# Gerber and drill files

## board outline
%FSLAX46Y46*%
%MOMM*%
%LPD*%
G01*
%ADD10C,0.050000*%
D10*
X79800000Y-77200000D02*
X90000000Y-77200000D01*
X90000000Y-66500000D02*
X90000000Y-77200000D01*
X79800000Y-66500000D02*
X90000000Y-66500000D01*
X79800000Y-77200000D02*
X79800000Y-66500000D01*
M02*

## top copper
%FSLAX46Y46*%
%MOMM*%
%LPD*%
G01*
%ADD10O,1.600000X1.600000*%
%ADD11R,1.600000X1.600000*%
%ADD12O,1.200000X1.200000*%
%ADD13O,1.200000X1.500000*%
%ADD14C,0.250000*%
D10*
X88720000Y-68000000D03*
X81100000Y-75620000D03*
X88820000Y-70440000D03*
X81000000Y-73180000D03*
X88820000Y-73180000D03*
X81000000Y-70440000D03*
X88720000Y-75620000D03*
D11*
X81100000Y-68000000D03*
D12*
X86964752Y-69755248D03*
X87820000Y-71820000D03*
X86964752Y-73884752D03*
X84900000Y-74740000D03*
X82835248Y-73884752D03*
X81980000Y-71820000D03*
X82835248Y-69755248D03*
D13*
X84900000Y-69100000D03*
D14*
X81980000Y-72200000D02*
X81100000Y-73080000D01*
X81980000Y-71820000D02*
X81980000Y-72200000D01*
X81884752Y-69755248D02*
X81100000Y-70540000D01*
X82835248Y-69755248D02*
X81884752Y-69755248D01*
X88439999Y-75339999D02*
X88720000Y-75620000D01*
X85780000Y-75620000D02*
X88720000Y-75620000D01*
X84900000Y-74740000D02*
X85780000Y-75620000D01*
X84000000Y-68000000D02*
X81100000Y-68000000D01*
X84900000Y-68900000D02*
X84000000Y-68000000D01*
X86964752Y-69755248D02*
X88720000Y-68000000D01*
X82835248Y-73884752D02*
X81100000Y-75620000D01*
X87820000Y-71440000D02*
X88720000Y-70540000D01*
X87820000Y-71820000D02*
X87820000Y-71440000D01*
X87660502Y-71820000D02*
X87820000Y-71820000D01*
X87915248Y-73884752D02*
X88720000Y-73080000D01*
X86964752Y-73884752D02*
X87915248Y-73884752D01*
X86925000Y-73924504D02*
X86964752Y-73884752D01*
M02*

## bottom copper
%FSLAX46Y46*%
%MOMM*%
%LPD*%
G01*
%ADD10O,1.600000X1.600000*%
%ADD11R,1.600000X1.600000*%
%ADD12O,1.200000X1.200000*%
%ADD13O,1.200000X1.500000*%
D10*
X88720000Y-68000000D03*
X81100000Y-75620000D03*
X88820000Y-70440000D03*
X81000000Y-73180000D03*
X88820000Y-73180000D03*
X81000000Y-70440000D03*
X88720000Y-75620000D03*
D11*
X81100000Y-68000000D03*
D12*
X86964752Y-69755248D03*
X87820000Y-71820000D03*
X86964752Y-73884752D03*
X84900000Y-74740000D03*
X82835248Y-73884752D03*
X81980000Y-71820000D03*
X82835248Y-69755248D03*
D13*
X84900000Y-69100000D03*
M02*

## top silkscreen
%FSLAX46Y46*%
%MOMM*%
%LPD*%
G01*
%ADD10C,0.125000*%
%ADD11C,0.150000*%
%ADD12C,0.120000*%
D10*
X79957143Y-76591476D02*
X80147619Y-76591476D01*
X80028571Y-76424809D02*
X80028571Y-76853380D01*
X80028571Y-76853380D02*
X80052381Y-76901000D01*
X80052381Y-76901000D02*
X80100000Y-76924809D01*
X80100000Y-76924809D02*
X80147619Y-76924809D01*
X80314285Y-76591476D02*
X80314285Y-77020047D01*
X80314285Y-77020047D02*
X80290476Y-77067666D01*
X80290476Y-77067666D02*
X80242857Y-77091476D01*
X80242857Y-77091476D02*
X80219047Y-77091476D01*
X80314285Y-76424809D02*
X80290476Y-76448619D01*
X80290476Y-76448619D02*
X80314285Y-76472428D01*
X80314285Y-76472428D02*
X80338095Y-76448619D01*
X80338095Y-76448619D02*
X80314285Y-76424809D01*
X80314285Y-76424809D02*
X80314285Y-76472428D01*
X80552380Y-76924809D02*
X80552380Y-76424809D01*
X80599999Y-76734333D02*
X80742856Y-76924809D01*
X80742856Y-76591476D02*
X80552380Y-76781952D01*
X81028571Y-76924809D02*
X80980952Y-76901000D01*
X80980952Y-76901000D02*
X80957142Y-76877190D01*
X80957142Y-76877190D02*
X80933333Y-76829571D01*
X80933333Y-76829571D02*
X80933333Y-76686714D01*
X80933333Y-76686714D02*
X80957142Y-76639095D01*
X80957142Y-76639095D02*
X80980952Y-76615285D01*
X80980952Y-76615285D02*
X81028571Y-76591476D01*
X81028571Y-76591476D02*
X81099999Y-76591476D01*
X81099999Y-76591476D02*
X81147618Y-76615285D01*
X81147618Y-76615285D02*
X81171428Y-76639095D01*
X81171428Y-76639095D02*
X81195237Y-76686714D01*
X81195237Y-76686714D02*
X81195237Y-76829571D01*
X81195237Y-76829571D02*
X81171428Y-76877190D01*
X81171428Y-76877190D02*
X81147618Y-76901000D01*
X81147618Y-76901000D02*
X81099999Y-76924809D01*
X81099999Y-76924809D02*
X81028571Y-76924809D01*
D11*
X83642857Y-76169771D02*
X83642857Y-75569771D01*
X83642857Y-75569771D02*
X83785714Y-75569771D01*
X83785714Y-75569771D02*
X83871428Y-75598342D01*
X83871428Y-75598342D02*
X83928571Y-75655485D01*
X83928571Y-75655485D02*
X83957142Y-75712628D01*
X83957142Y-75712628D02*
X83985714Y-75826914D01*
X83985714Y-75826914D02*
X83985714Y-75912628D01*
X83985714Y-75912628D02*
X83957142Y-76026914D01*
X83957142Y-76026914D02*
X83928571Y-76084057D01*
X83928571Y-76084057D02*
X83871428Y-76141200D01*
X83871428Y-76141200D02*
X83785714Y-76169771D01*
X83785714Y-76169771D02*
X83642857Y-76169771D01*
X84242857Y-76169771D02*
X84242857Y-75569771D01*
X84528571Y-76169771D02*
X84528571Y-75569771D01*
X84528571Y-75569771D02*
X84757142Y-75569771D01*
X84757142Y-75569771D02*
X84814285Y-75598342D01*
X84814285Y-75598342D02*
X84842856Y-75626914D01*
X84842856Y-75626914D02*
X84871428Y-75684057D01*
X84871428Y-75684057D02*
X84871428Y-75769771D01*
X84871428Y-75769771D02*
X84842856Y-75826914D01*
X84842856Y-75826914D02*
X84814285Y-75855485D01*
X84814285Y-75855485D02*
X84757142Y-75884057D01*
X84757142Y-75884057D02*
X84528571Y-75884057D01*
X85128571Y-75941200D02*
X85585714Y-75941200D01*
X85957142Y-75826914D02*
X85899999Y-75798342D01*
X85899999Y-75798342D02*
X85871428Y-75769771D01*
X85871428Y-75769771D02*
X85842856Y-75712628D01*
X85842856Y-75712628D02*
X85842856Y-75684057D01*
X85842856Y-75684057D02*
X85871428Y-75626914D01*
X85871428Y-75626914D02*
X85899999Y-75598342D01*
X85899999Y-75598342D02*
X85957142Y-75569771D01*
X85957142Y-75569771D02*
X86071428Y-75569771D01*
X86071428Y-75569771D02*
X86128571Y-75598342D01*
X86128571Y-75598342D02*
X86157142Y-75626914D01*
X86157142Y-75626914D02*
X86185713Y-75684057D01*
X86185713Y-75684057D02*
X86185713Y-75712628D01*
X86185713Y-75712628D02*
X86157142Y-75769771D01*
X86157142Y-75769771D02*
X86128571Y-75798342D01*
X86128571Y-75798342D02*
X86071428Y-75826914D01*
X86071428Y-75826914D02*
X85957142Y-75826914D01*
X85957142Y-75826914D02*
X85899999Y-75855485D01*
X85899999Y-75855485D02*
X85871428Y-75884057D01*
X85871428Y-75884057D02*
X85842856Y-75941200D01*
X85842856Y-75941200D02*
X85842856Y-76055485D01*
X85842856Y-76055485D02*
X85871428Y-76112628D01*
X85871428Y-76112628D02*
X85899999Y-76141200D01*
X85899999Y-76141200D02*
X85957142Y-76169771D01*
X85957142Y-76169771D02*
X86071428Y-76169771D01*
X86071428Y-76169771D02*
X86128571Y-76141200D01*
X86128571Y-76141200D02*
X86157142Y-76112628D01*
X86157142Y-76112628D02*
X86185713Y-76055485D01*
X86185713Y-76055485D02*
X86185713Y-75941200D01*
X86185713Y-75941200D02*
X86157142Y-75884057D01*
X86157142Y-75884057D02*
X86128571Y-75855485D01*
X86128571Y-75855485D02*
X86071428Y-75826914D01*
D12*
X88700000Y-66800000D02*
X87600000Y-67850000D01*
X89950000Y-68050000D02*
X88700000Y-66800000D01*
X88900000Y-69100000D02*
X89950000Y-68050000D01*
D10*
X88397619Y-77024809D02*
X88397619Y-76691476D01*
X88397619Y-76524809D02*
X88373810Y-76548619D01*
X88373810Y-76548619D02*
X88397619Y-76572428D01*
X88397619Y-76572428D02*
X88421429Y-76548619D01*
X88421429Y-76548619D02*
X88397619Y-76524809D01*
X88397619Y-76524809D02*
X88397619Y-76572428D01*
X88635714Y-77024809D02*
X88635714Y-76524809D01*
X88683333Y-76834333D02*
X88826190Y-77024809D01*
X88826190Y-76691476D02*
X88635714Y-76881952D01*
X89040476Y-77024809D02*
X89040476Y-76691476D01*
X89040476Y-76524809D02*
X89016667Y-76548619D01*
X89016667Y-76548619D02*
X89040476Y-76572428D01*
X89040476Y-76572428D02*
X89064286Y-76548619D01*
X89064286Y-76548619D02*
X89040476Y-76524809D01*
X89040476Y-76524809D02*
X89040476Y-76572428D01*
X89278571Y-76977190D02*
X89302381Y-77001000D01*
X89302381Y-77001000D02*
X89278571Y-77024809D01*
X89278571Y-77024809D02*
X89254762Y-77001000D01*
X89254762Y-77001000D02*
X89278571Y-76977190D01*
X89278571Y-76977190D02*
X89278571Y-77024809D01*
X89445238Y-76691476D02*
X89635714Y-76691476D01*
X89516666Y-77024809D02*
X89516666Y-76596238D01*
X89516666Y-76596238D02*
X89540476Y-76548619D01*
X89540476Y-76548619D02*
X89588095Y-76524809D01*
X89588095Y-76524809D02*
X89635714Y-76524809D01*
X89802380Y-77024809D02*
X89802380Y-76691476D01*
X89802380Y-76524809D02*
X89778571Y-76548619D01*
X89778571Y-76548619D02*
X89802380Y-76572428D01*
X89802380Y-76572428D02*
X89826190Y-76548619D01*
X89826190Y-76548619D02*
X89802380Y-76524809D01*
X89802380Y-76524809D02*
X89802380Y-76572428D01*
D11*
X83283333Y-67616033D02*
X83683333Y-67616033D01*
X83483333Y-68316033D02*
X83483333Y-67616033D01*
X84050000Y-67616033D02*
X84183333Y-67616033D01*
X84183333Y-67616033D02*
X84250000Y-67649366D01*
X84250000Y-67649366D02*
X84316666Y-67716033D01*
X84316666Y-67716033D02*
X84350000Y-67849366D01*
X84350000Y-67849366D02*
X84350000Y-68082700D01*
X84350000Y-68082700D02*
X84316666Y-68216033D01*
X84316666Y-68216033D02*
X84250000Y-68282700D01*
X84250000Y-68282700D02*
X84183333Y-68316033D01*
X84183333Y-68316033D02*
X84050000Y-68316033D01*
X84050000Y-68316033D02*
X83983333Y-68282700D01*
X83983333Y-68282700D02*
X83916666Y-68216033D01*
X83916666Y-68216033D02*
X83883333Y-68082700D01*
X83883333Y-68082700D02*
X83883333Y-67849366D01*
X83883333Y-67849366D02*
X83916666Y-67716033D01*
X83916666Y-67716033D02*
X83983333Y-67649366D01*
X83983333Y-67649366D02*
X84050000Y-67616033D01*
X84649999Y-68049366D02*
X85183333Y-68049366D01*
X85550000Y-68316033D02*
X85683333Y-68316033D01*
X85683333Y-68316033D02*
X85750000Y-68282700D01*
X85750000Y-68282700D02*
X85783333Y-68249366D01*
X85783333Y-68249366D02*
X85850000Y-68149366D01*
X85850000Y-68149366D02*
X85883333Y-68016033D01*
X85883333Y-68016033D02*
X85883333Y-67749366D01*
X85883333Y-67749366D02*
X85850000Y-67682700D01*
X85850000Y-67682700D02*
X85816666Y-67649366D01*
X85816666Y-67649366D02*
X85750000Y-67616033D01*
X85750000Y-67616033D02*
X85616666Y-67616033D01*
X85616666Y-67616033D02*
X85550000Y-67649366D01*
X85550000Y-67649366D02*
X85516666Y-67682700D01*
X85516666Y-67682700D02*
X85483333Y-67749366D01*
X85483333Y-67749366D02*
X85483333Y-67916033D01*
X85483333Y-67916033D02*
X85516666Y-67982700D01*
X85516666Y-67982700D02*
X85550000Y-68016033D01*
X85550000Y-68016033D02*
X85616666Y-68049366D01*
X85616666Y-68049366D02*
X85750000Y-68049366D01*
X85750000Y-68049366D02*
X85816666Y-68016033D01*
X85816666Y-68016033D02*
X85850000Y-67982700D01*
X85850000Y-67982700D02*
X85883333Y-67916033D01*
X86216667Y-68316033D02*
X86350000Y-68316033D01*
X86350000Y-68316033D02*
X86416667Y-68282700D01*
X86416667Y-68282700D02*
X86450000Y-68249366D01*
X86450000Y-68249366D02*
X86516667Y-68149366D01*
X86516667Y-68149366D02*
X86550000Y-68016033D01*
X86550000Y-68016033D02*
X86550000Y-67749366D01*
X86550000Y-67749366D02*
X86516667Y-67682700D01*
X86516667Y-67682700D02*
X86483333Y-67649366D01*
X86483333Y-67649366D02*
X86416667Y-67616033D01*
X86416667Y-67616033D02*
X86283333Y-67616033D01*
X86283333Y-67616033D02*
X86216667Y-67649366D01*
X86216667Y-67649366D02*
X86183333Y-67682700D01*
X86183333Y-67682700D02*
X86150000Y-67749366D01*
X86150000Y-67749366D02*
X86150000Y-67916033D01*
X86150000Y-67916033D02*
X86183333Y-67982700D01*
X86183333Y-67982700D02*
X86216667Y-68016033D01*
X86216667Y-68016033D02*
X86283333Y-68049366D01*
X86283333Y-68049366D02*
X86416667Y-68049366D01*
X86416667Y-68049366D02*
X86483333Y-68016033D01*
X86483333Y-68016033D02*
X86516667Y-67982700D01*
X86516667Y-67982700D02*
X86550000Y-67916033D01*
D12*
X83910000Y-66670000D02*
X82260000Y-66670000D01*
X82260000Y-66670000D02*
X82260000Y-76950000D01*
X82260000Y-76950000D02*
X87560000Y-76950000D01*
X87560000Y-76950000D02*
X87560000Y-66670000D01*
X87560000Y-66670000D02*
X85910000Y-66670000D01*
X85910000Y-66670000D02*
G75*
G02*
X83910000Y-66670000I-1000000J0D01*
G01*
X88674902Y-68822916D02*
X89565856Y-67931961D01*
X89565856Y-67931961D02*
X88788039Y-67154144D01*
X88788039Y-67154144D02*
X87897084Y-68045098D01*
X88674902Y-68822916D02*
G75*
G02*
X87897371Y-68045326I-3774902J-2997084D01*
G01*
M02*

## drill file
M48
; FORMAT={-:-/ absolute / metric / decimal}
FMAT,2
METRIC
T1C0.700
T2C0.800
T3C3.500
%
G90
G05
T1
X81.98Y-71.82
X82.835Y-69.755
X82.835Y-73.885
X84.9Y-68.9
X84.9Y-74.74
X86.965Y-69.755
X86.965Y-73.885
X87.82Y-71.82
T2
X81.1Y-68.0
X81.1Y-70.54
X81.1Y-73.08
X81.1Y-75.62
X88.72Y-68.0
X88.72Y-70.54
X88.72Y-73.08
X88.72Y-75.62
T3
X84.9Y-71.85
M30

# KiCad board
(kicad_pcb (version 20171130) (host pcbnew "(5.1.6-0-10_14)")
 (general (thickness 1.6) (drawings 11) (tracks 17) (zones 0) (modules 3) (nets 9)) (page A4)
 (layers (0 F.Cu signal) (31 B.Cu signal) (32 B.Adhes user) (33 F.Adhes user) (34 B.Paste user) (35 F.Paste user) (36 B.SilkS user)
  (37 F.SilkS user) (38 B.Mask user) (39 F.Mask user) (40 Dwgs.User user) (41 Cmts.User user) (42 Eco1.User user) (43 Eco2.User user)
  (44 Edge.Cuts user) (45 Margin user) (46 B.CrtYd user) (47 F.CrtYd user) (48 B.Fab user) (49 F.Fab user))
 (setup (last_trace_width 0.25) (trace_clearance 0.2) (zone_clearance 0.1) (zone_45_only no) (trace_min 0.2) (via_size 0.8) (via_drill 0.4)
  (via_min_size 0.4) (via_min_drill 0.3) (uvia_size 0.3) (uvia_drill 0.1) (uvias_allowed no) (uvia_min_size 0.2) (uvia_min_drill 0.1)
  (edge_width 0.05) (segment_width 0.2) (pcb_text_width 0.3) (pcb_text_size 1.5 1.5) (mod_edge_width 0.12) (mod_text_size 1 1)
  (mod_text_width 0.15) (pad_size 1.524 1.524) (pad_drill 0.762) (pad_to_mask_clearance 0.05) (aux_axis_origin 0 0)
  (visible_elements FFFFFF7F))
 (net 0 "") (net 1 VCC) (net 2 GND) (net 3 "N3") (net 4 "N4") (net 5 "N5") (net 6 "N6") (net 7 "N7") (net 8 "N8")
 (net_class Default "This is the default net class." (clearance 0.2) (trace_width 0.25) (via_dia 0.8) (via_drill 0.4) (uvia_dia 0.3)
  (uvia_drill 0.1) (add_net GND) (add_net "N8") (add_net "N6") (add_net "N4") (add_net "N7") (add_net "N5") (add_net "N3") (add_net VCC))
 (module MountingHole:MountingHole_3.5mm (layer F.Cu) (at 84.9 71.85)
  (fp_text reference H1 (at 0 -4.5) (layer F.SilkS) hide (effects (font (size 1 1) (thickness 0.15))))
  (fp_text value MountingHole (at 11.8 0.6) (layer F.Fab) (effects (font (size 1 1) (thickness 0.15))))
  (pad 1 np_thru_hole circle (at 0 0) (size 3.5 3.5) (drill 3.5) (layers *.Cu *.Mask)))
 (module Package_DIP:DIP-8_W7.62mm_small (layer F.Cu) (at 81.1 68)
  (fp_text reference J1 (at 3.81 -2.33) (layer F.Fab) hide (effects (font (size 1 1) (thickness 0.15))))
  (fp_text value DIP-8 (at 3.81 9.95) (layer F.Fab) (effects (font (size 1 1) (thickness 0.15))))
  (fp_line (start 2.81 -1.33) (end 1.16 -1.33) (layer F.SilkS) (width 0.12))
  (fp_line (start 1.16 -1.33) (end 1.16 8.95) (layer F.SilkS) (width 0.12))
  (fp_line (start 1.16 8.95) (end 6.46 8.95) (layer F.SilkS) (width 0.12))
  (fp_line (start 6.46 8.95) (end 6.46 -1.33) (layer F.SilkS) (width 0.12))
  (fp_line (start 6.46 -1.33) (end 4.81 -1.33) (layer F.SilkS) (width 0.12))
  (fp_arc (start 3.81 -1.33) (end 2.81 -1.33) (angle -180) (layer F.SilkS) (width 0.12))
  (pad 8 thru_hole oval (at 7.62 0) (size 1.6 1.6) (drill 0.8) (layers *.Cu *.Mask) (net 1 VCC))
  (pad 4 thru_hole oval (at 0 7.62) (size 1.6 1.6) (drill 0.8) (layers *.Cu *.Mask) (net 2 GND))
  (pad 7 thru_hole oval (at 7.62 2.54) (size 1.6 1.6) (drill 0.8 (offset 0.1 -0.1)) (layers *.Cu *.Mask) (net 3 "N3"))
  (pad 3 thru_hole oval (at 0 5.08) (size 1.6 1.6) (drill 0.8 (offset -0.1 0.1)) (layers *.Cu *.Mask) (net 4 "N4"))
  (pad 6 thru_hole oval (at 7.62 5.08) (size 1.6 1.6) (drill 0.8 (offset 0.1 0.1)) (layers *.Cu *.Mask) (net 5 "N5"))
  (pad 2 thru_hole oval (at 0 2.54) (size 1.6 1.6) (drill 0.8 (offset -0.1 -0.1)) (layers *.Cu *.Mask) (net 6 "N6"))
  (pad 5 thru_hole oval (at 7.62 7.62) (size 1.6 1.6) (drill 0.8) (layers *.Cu *.Mask) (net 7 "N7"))
  (pad 1 thru_hole rect (at 0 0) (size 1.6 1.6) (drill 0.8) (layers *.Cu *.Mask) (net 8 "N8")))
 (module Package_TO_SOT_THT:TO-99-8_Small (layer F.Cu) (at 84.9 68.9 270)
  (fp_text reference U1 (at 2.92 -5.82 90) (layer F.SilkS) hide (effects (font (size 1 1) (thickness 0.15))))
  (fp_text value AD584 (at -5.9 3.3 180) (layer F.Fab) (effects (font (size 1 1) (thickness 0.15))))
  (fp_line (start -0.077084 -3.774902) (end -0.968039 -4.665856) (layer F.SilkS) (width 0.12))
  (fp_line (start -0.968039 -4.665856) (end -1.745856 -3.888039) (layer F.SilkS) (width 0.12))
  (fp_line (start -1.745856 -3.888039) (end -0.854902 -2.997084) (layer F.SilkS) (width 0.12))
  (fp_arc (start 2.92 0) (end -0.077084 -3.774902) (angle 346.9) (layer F.SilkS) (width 0.12))
  (pad 8 thru_hole oval (at 0.855248 -2.064752 270) (size 1.2 1.2) (drill 0.7) (layers *.Cu *.Mask) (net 1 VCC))
  (pad 7 thru_hole oval (at 2.92 -2.92 270) (size 1.2 1.2) (drill 0.7) (layers *.Cu *.Mask) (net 3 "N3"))
  (pad 6 thru_hole oval (at 4.984752 -2.064752 270) (size 1.2 1.2) (drill 0.7) (layers *.Cu *.Mask) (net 5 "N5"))
  (pad 5 thru_hole oval (at 5.84 0 270) (size 1.2 1.2) (drill 0.7) (layers *.Cu *.Mask) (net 7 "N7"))
  (pad 4 thru_hole oval (at 4.984752 2.064752 270) (size 1.2 1.2) (drill 0.7) (layers *.Cu *.Mask) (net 2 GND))
  (pad 3 thru_hole oval (at 2.92 2.92 270) (size 1.2 1.2) (drill 0.7) (layers *.Cu *.Mask) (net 4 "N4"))
  (pad 2 thru_hole oval (at 0.855248 2.064752 270) (size 1.2 1.2) (drill 0.7) (layers *.Cu *.Mask) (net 6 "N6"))
  (pad 1 thru_hole oval (at 0 0 270) (size 1.5 1.2) (drill 0.7 (offset 0.2 0)) (layers *.Cu *.Mask) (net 8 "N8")))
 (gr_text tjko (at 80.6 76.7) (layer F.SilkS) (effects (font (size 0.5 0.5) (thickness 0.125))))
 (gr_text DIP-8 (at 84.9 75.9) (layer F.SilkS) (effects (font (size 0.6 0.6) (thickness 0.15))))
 (gr_line (start 88.7 66.8) (end 87.6 67.85) (layer F.SilkS) (width 0.12))
 (gr_line (start 89.95 68.05) (end 88.7 66.8) (layer F.SilkS) (width 0.12))
 (gr_line (start 88.9 69.1) (end 89.95 68.05) (layer F.SilkS) (width 0.12))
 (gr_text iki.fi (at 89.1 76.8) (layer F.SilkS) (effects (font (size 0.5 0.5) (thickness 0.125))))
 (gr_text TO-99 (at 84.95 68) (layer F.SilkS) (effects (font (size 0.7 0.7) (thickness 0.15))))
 (gr_line (start 79.8 77.2) (end 90 77.2) (layer Edge.Cuts) (width 0.05))
 (gr_line (start 90 66.5) (end 90 77.2) (layer Edge.Cuts) (width 0.05))
 (gr_line (start 79.8 66.5) (end 90 66.5) (layer Edge.Cuts) (width 0.05))
 (gr_line (start 79.8 77.2) (end 79.8 66.5) (layer Edge.Cuts) (width 0.05))
 (segment (start 81.98 72.2) (end 81.1 73.08) (width 0.25) (layer F.Cu) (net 4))
 (segment (start 81.98 71.82) (end 81.98 72.2) (width 0.25) (layer F.Cu) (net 4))
 (segment (start 81.884752 69.755248) (end 81.1 70.54) (width 0.25) (layer F.Cu) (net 6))
 (segment (start 82.835248 69.755248) (end 81.884752 69.755248) (width 0.25) (layer F.Cu) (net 6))
 (segment (start 88.439999 75.339999) (end 88.72 75.62) (width 0.25) (layer F.Cu) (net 7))
 (segment (start 85.78 75.62) (end 88.72 75.62) (width 0.25) (layer F.Cu) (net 7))
 (segment (start 84.9 74.74) (end 85.78 75.62) (width 0.25) (layer F.Cu) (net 7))
 (segment (start 84 68) (end 81.1 68) (width 0.25) (layer F.Cu) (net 8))
 (segment (start 84.9 68.9) (end 84 68) (width 0.25) (layer F.Cu) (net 8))
 (segment (start 86.964752 69.755248) (end 88.72 68) (width 0.25) (layer F.Cu) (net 1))
 (segment (start 82.835248 73.884752) (end 81.1 75.62) (width 0.25) (layer F.Cu) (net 2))
 (segment (start 87.82 71.44) (end 88.72 70.54) (width 0.25) (layer F.Cu) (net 3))
 (segment (start 87.82 71.82) (end 87.82 71.44) (width 0.25) (layer F.Cu) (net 3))
 (segment (start 87.660502 71.82) (end 87.82 71.82) (width 0.25) (layer F.Cu) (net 3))
 (segment (start 87.915248 73.884752) (end 88.72 73.08) (width 0.25) (layer F.Cu) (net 5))
 (segment (start 86.964752 73.884752) (end 87.915248 73.884752) (width 0.25) (layer F.Cu) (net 5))
 (segment (start 86.925 73.924504) (end 86.964752 73.884752) (width 0.25) (layer F.Cu) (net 5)))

